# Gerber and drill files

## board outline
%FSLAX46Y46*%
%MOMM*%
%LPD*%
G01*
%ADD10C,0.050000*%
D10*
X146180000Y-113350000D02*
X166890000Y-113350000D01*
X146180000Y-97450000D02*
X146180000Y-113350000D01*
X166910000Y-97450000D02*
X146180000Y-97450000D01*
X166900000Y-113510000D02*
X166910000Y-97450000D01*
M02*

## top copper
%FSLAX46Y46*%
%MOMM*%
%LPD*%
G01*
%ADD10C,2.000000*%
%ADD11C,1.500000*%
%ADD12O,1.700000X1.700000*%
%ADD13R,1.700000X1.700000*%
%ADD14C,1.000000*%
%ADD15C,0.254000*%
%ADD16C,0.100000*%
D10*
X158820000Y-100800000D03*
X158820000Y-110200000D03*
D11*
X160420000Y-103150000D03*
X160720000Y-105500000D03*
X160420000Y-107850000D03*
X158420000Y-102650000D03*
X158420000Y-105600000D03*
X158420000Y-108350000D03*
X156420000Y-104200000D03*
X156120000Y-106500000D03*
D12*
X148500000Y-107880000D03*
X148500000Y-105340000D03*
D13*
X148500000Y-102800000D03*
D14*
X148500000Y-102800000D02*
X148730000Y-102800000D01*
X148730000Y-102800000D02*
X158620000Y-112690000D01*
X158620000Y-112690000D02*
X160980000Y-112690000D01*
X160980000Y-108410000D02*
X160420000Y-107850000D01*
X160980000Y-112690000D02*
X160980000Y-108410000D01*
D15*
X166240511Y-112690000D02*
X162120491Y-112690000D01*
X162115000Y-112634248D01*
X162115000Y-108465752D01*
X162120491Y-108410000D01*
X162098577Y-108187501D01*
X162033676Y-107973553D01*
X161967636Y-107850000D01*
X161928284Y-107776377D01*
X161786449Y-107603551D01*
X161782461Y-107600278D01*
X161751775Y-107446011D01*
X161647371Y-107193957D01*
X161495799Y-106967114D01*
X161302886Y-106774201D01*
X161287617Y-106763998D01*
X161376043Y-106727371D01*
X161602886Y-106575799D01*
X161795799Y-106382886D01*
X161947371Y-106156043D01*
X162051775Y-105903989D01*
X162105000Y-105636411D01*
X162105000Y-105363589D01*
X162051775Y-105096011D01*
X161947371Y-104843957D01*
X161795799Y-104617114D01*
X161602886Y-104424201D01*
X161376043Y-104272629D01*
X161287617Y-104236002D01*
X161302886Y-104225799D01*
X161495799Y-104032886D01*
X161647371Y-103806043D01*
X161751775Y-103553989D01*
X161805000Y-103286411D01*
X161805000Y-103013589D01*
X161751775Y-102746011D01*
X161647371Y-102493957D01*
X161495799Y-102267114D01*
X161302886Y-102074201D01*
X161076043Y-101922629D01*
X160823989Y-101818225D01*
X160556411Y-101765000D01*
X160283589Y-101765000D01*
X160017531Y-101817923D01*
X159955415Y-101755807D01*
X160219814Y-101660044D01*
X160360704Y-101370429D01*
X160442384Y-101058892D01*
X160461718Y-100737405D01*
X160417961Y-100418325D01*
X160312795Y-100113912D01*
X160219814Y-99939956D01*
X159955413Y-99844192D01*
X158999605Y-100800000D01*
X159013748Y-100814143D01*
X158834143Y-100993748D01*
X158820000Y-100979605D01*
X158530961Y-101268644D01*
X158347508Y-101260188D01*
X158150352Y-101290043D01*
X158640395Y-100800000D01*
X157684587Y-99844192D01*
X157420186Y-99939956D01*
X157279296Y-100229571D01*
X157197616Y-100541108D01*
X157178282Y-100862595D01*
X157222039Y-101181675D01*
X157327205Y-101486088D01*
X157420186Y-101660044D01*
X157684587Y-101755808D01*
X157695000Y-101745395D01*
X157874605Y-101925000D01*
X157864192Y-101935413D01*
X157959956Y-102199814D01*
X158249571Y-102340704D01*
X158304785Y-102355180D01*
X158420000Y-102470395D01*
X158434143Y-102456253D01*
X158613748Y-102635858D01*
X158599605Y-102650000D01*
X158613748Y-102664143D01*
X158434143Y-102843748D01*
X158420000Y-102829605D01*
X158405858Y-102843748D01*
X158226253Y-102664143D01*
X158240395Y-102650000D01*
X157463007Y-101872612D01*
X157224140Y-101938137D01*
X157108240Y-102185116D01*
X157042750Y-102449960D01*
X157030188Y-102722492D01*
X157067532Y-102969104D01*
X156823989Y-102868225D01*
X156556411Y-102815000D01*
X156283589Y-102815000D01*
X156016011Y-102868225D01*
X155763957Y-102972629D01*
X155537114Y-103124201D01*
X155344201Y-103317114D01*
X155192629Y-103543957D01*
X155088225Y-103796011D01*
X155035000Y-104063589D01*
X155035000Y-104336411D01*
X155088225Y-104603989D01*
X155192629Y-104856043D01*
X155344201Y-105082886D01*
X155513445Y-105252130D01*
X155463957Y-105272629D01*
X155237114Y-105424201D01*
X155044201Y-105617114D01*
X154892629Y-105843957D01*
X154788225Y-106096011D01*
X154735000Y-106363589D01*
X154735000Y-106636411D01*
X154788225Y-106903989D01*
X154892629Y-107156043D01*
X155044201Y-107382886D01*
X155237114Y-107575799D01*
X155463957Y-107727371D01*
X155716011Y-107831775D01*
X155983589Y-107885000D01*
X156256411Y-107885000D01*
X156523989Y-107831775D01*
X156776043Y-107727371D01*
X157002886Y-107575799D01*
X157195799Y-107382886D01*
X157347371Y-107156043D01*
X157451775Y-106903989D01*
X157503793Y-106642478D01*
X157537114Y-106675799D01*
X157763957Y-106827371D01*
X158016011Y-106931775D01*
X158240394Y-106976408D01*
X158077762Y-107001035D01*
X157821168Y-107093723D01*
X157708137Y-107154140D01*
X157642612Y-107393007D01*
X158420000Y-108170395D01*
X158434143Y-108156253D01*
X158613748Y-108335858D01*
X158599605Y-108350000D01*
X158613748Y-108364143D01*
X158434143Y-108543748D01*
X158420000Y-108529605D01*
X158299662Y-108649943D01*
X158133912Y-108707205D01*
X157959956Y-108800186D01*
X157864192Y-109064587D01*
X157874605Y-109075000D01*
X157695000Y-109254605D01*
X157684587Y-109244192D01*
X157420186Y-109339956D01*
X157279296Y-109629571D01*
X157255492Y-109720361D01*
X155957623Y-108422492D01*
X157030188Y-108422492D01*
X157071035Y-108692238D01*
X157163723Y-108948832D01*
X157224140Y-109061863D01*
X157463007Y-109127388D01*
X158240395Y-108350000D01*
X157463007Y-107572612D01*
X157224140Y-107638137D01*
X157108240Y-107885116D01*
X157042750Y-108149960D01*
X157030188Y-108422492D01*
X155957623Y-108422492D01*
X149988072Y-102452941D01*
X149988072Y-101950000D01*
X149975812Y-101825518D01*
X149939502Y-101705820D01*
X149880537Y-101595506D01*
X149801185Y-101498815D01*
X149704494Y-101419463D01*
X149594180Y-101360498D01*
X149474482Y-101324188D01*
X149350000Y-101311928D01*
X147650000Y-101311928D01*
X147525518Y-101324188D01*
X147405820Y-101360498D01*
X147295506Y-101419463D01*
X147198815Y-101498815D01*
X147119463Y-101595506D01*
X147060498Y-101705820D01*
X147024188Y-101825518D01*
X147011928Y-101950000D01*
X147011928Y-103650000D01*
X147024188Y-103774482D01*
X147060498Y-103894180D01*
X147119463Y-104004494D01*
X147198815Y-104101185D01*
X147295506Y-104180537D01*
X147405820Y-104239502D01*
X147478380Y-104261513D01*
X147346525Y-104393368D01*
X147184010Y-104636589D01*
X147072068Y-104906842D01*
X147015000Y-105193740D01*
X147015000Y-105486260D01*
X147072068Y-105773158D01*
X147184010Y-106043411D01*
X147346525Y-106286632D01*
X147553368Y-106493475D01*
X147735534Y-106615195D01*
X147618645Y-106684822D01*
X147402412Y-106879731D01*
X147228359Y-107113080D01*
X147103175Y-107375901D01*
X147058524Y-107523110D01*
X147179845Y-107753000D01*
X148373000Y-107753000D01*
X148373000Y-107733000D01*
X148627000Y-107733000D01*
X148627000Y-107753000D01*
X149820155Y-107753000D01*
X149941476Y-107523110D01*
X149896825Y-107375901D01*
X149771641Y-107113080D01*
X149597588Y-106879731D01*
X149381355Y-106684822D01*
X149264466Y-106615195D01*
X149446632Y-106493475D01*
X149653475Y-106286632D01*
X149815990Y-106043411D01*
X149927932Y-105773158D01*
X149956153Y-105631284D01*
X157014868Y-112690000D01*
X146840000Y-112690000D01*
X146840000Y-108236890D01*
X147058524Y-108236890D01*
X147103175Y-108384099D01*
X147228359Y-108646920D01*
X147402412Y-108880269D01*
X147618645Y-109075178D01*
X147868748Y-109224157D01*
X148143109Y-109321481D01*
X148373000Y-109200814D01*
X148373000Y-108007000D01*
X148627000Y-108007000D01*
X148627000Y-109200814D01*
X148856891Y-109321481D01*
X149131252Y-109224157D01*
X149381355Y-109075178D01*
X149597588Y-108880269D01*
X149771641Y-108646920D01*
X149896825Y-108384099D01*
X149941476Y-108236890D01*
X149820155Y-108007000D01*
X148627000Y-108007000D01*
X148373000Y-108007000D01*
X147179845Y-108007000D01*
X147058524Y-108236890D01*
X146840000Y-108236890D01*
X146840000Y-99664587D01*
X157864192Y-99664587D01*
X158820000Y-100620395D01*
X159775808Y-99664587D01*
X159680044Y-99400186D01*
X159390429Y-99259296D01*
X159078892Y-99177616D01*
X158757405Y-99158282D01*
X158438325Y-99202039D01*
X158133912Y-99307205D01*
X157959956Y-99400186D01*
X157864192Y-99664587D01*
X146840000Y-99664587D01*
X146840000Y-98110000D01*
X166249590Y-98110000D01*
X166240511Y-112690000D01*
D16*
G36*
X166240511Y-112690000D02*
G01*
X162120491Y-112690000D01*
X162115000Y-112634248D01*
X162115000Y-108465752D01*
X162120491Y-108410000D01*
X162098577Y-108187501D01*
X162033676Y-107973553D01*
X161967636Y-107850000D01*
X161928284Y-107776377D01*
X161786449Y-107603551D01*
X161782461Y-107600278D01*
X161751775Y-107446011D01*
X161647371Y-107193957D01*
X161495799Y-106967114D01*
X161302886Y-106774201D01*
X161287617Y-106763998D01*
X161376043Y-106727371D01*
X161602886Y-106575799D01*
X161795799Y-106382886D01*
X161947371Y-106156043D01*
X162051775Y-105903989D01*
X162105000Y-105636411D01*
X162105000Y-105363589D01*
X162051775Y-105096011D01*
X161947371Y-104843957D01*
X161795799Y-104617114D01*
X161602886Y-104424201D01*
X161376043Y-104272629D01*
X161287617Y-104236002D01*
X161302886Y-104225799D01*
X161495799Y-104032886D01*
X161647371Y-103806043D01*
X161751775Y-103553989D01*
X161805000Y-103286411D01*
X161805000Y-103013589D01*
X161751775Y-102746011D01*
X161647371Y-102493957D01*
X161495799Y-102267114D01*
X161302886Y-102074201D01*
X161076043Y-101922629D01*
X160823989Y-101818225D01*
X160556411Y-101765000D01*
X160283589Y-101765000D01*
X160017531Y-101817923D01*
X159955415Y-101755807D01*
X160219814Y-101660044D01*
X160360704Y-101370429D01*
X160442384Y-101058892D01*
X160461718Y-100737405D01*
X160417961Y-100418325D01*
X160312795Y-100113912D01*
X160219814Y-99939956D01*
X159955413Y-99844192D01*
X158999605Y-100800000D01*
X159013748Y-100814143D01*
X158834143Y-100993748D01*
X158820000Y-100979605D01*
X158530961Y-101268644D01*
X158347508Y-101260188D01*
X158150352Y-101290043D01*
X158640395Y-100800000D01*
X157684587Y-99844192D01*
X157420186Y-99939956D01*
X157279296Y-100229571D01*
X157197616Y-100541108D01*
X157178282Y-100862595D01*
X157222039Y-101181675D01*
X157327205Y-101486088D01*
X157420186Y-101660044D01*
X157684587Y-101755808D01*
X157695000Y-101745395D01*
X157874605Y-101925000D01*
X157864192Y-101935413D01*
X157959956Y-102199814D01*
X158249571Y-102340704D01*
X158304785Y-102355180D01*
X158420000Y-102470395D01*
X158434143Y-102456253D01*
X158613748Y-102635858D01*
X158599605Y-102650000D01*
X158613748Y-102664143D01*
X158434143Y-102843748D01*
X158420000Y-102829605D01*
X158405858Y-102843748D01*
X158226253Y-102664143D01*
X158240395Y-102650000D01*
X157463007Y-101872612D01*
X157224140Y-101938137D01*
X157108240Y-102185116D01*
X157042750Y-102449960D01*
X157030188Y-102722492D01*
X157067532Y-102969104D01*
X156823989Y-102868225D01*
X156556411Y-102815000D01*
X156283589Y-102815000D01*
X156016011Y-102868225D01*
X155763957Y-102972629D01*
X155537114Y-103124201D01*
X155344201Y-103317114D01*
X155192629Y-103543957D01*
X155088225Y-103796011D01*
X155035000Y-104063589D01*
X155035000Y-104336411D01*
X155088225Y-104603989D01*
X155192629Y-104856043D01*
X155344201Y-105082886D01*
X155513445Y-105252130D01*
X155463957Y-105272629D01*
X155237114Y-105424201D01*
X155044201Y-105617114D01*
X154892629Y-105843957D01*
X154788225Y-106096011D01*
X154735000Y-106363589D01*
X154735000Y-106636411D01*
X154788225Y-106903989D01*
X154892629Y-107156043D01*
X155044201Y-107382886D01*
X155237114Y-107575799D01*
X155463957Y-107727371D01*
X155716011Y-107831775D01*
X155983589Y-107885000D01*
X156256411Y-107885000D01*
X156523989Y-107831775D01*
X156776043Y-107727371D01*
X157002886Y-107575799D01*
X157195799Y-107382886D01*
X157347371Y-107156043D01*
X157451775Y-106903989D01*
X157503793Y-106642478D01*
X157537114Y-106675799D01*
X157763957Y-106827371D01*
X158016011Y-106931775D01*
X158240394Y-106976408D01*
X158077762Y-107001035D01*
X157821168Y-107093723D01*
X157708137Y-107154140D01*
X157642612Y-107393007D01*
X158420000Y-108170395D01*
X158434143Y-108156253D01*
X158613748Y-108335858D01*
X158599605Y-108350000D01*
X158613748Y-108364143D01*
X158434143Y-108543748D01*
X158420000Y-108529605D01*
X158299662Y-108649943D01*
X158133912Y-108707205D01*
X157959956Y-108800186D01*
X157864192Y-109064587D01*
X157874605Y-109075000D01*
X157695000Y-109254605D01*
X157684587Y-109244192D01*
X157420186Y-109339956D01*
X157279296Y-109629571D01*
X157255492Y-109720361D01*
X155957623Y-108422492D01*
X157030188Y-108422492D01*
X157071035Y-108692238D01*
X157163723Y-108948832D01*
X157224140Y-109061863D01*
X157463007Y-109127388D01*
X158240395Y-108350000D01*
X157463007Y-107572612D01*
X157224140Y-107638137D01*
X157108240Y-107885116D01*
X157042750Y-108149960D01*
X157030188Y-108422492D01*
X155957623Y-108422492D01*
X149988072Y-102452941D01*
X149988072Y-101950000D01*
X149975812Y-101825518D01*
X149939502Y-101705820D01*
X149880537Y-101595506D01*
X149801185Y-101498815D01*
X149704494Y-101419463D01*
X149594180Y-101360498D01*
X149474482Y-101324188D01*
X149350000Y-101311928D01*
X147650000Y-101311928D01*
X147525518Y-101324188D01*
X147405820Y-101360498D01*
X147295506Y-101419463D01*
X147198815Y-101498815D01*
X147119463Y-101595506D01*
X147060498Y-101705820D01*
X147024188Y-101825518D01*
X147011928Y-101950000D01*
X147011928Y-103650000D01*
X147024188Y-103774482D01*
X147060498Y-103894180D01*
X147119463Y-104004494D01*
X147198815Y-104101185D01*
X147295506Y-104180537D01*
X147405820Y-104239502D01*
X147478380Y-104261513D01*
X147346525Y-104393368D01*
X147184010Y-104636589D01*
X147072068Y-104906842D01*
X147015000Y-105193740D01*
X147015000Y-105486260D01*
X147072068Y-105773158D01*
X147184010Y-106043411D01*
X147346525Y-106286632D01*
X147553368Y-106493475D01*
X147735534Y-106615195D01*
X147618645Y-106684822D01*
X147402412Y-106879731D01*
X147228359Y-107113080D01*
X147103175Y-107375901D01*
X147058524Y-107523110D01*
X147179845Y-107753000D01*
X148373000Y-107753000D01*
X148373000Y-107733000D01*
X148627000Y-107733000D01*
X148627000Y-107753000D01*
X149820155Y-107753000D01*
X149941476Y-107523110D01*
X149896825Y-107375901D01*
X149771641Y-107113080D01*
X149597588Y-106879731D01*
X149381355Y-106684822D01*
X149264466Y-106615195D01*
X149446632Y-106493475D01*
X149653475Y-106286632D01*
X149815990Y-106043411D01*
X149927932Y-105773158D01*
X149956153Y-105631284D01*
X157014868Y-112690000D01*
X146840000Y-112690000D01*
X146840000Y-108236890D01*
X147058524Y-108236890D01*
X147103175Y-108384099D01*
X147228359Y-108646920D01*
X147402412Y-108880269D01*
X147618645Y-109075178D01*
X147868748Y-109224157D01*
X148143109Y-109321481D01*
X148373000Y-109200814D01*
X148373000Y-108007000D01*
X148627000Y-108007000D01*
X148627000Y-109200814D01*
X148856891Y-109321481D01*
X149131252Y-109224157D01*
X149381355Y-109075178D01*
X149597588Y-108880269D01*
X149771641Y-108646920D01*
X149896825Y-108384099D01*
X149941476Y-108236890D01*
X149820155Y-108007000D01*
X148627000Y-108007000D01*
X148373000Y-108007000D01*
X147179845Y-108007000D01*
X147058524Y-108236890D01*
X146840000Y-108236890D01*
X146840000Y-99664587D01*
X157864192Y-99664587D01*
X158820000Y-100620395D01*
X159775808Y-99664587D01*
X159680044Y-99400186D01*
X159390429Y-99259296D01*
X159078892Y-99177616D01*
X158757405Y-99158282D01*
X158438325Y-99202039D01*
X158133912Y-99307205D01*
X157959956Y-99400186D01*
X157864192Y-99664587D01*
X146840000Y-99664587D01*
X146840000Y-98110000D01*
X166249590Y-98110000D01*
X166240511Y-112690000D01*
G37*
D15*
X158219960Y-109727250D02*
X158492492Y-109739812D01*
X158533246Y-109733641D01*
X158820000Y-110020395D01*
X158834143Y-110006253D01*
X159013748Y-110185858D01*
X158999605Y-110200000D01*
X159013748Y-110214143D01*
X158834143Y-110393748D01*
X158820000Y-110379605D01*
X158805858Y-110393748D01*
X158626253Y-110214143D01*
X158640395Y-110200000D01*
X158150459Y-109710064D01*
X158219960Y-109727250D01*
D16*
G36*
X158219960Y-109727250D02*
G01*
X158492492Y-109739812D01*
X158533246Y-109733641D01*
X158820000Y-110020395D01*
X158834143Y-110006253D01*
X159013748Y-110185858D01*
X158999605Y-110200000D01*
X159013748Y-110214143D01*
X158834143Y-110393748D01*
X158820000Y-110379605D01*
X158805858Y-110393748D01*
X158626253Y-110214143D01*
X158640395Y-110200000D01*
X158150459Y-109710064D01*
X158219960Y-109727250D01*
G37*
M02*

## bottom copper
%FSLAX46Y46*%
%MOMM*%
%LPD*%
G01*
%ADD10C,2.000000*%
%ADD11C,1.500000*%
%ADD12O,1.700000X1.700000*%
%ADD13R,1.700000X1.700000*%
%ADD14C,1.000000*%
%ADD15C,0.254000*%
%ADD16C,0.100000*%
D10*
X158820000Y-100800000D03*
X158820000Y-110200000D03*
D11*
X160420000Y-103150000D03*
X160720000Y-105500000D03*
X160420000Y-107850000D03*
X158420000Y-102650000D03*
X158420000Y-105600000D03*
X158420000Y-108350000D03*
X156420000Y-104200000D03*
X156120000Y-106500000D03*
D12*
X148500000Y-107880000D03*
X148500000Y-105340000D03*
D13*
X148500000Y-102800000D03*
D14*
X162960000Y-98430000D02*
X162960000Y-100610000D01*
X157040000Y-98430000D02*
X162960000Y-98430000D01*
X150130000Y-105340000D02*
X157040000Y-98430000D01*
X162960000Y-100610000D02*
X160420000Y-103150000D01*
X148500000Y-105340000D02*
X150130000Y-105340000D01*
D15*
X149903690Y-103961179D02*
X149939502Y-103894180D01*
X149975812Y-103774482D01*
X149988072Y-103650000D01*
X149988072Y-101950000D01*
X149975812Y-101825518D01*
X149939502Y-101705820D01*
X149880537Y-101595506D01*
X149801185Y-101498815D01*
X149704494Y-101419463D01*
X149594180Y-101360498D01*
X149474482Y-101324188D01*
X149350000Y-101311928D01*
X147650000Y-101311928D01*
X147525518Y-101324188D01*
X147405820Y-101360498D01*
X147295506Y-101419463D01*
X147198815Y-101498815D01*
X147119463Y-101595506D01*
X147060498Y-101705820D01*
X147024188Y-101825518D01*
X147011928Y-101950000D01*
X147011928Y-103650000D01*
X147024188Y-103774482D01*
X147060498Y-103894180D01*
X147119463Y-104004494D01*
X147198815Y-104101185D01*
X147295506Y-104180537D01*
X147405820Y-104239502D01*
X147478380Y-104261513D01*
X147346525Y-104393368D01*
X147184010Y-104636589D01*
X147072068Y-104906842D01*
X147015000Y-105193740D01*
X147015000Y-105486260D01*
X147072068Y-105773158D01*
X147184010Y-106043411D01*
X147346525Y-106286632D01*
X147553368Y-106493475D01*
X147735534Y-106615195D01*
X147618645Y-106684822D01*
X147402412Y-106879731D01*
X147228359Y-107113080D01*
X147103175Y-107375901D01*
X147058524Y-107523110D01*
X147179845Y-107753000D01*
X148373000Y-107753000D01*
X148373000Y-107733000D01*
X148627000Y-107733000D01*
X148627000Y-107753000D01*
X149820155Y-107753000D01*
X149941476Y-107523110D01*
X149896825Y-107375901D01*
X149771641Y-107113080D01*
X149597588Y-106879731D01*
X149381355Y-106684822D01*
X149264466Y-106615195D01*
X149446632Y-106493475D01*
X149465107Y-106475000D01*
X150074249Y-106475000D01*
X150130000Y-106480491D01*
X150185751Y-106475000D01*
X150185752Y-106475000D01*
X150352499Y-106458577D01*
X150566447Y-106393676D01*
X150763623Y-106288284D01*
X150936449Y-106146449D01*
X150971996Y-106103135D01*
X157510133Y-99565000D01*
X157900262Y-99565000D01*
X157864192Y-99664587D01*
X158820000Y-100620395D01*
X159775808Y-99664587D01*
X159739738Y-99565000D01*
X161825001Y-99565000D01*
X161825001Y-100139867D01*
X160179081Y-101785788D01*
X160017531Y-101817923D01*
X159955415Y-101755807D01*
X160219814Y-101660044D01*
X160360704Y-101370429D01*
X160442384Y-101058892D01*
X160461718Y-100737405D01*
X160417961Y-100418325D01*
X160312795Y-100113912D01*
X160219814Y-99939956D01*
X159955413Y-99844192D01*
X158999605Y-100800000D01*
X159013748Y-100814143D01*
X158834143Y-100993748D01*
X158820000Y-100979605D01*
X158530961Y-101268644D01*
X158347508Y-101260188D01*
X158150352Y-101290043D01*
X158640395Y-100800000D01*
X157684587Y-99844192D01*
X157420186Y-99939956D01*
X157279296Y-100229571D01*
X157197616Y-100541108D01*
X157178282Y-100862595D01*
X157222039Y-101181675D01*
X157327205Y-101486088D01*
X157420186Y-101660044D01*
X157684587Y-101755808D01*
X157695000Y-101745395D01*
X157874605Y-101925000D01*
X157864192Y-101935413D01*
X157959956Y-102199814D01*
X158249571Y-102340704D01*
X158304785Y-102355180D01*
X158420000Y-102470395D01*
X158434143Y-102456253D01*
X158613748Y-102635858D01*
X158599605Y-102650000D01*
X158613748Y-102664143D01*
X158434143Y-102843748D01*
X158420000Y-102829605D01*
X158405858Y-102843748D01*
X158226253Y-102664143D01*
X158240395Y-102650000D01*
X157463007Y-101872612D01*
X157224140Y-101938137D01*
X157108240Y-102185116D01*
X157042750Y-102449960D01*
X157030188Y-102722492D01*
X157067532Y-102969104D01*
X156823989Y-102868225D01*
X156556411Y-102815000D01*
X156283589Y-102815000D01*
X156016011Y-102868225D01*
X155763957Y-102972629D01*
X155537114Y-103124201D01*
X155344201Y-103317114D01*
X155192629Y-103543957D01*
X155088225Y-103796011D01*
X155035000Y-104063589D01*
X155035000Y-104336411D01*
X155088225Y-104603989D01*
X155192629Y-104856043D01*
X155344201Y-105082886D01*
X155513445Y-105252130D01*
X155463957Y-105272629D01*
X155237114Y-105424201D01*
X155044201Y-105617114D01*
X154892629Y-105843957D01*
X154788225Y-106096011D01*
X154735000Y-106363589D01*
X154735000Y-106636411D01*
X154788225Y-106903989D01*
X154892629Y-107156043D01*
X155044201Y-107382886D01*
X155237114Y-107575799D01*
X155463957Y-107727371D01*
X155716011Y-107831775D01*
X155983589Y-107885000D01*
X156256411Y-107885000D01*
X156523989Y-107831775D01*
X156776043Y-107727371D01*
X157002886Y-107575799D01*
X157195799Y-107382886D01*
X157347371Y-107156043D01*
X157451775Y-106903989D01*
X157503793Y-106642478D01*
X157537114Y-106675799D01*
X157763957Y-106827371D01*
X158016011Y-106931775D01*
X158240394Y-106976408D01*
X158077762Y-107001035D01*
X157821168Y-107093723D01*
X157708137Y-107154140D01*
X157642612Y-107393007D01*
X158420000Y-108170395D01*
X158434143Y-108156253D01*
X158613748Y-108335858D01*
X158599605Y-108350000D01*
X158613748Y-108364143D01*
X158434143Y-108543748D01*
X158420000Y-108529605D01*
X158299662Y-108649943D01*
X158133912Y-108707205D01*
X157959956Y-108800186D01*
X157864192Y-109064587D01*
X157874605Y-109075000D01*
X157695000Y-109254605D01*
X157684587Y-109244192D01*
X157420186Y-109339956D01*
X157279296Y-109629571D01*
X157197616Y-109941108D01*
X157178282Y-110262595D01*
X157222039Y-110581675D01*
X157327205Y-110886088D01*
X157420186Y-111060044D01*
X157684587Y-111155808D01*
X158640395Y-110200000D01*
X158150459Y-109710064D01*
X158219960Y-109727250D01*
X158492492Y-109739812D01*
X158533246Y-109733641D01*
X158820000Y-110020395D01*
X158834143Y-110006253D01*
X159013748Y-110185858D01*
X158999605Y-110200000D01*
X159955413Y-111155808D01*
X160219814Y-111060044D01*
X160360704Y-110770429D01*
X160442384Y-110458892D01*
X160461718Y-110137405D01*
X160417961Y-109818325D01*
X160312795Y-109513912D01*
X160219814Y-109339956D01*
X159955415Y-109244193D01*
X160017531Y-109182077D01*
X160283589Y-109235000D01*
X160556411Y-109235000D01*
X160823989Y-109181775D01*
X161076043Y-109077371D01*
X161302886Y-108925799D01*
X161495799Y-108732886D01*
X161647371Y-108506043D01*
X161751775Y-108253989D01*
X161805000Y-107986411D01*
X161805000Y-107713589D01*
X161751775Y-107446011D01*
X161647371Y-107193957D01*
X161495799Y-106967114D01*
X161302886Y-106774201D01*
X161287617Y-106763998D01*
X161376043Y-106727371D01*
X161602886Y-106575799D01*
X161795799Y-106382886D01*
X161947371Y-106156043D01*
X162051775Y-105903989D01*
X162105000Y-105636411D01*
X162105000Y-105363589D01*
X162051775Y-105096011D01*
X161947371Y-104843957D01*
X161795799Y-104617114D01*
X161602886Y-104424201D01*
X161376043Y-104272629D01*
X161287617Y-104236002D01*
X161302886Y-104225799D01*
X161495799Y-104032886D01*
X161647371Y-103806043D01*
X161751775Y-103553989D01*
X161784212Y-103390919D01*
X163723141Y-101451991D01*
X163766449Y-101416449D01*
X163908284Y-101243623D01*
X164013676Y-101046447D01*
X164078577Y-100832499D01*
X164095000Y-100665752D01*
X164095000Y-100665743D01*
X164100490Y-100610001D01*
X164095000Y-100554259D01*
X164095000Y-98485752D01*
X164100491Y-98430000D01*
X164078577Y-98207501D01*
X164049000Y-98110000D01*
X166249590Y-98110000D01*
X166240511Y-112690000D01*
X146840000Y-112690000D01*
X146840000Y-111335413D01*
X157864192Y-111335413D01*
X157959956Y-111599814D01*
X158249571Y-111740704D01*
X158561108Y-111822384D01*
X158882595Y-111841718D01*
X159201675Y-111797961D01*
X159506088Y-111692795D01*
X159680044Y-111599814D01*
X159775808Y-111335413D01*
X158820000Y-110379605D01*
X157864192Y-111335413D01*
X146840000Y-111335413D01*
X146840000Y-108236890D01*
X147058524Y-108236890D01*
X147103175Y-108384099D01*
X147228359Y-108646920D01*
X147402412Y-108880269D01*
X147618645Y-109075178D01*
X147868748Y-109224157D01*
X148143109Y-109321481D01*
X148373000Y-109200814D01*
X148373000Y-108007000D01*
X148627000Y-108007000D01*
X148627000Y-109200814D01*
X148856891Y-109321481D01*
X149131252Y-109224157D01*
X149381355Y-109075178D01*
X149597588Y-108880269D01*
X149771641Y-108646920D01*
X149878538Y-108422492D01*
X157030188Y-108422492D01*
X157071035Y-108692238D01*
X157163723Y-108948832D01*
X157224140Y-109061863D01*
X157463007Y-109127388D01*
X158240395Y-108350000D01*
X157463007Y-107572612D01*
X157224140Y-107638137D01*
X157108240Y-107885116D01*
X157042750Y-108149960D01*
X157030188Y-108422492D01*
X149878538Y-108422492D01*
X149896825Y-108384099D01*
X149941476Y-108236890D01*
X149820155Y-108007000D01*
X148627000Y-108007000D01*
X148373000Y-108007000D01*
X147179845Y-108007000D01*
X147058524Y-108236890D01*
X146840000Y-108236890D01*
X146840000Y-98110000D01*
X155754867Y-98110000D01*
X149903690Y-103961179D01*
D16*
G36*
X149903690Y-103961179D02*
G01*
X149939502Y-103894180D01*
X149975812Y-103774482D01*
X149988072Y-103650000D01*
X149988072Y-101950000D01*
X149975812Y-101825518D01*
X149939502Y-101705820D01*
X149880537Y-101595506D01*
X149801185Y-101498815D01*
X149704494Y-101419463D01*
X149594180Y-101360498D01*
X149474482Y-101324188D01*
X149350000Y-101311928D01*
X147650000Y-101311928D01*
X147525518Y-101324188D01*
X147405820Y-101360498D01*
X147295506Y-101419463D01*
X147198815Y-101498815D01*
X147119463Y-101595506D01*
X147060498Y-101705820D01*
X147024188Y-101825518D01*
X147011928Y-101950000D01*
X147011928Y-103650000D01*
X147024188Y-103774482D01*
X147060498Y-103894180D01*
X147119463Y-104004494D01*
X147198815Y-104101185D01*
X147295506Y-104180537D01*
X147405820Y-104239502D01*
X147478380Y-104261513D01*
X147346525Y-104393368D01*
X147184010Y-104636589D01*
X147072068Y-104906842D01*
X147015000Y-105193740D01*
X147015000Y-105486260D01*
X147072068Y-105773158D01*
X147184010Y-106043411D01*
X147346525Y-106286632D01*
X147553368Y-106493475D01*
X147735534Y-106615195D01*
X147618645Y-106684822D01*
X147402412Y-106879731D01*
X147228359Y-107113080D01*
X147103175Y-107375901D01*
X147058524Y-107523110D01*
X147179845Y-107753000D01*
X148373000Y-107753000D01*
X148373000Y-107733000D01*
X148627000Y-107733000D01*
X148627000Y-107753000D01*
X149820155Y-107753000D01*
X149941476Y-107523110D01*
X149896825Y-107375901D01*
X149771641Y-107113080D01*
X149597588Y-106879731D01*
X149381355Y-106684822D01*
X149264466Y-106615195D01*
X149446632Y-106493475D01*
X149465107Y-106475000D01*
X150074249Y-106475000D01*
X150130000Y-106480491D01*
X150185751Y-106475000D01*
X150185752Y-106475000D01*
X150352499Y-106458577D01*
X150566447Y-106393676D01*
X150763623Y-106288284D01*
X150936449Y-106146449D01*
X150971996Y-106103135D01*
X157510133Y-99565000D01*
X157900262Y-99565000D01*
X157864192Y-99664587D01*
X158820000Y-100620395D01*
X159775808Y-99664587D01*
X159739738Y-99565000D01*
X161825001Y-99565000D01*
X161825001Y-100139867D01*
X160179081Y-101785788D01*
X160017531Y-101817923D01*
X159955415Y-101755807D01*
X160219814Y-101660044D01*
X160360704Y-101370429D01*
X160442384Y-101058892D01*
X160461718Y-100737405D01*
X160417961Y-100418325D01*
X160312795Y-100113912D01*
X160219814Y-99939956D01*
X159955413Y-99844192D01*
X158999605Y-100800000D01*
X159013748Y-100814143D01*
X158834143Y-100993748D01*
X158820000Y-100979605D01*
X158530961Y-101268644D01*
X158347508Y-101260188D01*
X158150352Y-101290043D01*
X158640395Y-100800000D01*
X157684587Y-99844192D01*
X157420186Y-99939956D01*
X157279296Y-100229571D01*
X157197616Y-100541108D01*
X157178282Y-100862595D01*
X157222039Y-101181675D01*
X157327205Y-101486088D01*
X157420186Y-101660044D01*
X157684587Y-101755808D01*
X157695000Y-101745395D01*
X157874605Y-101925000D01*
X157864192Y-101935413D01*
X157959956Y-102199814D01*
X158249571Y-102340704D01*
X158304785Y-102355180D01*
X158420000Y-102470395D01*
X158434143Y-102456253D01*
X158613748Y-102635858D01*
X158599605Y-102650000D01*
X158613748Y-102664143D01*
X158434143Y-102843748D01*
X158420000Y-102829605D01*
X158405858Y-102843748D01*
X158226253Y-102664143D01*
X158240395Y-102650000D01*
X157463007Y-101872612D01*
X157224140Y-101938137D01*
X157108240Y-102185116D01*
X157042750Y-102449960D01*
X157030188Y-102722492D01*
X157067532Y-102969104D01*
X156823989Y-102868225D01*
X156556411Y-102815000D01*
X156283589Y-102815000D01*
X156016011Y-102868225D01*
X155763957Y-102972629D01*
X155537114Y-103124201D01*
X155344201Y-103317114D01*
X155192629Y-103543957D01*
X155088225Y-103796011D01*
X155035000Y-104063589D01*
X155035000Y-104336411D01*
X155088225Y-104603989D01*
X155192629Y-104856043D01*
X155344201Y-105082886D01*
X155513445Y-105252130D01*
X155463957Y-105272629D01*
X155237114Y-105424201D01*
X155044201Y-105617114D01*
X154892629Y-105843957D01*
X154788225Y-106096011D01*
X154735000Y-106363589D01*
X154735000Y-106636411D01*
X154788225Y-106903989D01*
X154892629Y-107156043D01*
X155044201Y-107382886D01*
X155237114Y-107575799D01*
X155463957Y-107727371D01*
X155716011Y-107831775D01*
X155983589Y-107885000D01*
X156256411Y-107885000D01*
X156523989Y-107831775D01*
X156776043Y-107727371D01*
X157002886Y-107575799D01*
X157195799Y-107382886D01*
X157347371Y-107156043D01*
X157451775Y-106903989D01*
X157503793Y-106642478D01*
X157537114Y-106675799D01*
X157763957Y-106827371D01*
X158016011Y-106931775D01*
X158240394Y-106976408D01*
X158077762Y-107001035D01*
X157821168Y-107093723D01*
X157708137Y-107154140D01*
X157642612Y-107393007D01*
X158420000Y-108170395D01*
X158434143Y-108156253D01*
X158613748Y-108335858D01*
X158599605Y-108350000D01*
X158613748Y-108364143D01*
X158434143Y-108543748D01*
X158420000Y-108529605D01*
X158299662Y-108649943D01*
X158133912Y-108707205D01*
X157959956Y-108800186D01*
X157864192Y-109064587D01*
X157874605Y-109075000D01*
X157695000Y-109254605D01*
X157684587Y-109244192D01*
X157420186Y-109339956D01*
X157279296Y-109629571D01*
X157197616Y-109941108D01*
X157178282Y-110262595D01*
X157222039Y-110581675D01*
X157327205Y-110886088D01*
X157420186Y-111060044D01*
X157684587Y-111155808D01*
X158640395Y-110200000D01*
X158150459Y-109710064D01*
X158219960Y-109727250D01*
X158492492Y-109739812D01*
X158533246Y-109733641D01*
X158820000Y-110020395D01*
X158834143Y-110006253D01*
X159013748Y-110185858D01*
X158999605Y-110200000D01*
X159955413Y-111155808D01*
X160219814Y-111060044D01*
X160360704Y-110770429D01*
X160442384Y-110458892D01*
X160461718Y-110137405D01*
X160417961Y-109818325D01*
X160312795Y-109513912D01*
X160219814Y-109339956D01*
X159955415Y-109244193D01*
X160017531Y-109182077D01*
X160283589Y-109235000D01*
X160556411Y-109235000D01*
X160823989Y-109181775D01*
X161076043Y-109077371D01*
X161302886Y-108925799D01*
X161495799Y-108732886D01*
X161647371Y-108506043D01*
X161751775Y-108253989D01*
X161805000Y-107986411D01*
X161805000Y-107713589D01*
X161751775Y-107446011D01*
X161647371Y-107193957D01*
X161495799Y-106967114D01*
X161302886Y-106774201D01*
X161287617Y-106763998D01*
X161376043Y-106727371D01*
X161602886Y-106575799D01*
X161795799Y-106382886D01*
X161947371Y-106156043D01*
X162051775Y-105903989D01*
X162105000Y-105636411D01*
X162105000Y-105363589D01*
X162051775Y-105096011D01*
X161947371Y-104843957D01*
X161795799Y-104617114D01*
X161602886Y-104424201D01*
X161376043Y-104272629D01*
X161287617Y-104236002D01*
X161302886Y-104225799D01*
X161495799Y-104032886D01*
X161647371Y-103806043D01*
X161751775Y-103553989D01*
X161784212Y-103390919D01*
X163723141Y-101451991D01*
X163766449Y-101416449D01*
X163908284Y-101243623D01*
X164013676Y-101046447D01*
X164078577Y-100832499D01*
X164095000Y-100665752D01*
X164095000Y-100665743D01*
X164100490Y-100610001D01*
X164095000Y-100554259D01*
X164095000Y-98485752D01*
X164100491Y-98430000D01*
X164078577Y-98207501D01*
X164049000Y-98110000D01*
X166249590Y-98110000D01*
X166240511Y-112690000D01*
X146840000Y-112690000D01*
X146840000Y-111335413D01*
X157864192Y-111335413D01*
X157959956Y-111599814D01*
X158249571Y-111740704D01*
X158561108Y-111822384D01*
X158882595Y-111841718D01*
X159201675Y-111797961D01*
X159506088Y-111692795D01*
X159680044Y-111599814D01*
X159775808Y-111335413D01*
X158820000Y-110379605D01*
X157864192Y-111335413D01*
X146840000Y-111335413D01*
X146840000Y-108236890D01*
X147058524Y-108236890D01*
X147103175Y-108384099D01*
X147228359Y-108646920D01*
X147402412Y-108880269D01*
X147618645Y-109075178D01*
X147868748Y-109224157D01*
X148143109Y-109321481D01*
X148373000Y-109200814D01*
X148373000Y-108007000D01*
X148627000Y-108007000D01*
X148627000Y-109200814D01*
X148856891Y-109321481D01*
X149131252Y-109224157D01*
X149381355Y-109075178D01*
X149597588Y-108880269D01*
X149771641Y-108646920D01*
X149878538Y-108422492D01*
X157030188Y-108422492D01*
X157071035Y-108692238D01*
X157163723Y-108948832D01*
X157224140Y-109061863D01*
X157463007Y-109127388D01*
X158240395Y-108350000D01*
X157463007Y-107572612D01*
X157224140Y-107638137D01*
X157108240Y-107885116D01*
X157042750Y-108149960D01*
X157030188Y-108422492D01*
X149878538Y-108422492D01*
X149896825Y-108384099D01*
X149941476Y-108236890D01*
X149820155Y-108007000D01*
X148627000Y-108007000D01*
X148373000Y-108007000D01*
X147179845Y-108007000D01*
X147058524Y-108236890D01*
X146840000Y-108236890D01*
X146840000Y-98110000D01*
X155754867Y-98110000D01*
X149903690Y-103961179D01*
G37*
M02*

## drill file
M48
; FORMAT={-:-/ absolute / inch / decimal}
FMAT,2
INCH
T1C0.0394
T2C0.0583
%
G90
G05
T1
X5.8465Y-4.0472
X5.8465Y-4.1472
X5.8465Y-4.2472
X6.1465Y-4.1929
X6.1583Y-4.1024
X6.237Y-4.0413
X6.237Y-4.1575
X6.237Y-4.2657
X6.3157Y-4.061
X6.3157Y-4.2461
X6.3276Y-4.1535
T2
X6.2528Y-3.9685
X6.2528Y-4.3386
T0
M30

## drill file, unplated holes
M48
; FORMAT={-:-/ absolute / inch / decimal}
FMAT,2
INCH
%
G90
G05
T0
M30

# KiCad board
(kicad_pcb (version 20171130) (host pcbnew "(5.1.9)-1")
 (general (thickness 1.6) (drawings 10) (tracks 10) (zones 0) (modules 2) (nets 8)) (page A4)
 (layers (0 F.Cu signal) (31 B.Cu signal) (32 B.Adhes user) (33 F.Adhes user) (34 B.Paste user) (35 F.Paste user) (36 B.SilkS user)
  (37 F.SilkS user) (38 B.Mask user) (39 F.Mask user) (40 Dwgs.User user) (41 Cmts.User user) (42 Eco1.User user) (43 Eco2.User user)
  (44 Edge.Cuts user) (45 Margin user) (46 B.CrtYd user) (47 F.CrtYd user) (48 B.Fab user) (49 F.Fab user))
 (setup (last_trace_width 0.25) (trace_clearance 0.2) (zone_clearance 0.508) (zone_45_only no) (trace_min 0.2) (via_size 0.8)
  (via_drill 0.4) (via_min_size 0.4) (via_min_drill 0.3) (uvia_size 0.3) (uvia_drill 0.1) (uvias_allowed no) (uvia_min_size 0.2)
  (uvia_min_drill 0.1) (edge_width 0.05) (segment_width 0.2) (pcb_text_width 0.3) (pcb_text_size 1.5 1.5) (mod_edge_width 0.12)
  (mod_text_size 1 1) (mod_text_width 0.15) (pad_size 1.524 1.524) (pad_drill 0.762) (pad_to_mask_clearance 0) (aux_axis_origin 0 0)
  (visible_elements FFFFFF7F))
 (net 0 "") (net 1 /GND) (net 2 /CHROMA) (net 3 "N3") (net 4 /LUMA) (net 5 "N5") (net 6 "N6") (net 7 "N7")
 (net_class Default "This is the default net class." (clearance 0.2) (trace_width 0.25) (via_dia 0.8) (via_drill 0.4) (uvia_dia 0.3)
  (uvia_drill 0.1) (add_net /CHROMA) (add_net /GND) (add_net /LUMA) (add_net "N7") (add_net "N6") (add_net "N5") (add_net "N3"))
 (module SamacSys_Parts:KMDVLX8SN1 (layer F.Cu) (at 156.12 106.5 90)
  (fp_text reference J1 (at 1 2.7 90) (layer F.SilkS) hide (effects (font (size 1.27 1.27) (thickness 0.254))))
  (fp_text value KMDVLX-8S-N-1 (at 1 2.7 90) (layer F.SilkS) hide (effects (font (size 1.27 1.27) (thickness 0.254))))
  (pad MH2 thru_hole circle (at 5.7 2.7 180) (size 2 2) (drill 1.48) (layers *.Cu *.Mask F.SilkS) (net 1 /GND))
  (pad MH1 thru_hole circle (at -3.7 2.7 180) (size 2 2) (drill 1.48) (layers *.Cu *.Mask F.SilkS) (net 1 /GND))
  (pad 8 thru_hole circle (at 3.35 4.3 180) (size 1.5 1.5) (drill 1) (layers *.Cu *.Mask F.SilkS) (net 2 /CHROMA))
  (pad 7 thru_hole circle (at 1 4.6 180) (size 1.5 1.5) (drill 1) (layers *.Cu *.Mask F.SilkS) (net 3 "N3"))
  (pad 6 thru_hole circle (at -1.35 4.3 180) (size 1.5 1.5) (drill 1) (layers *.Cu *.Mask F.SilkS) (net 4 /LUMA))
  (pad 5 thru_hole circle (at 3.85 2.3 180) (size 1.5 1.5) (drill 1) (layers *.Cu *.Mask F.SilkS) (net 1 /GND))
  (pad 4 thru_hole circle (at 0.9 2.3 180) (size 1.5 1.5) (drill 1) (layers *.Cu *.Mask F.SilkS) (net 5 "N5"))
  (pad 3 thru_hole circle (at -1.85 2.3 180) (size 1.5 1.5) (drill 1) (layers *.Cu *.Mask F.SilkS) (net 1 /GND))
  (pad 2 thru_hole circle (at 2.3 0.3 180) (size 1.5 1.5) (drill 1) (layers *.Cu *.Mask F.SilkS) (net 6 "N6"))
  (pad 1 thru_hole circle (at 0 0 180) (size 1.5 1.5) (drill 1) (layers *.Cu *.Mask F.SilkS) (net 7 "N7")))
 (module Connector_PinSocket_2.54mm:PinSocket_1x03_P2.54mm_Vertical (layer F.Cu) (at 148.5 102.8)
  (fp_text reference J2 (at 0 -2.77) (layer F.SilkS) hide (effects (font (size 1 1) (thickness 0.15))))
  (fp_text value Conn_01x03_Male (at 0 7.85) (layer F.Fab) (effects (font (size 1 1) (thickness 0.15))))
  (pad 3 thru_hole oval (at 0 5.08) (size 1.7 1.7) (drill 1) (layers *.Cu *.Mask) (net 1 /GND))
  (pad 2 thru_hole oval (at 0 2.54) (size 1.7 1.7) (drill 1) (layers *.Cu *.Mask) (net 2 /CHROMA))
  (pad 1 thru_hole rect (at 0 0) (size 1.7 1.7) (drill 1) (layers *.Cu *.Mask) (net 4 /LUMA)))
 (gr_line (start 146.18 113.35) (end 166.89 113.35) (layer Edge.Cuts) (width 0.05))
 (gr_line (start 146.18 97.45) (end 146.18 113.35) (layer Edge.Cuts) (width 0.05))
 (gr_line (start 166.91 97.45) (end 146.18 97.45) (layer Edge.Cuts) (width 0.05))
 (gr_line (start 166.9 113.51) (end 166.91 97.45) (layer Edge.Cuts) (width 0.05))
 (segment (start 162.96 98.43) (end 162.96 100.61) (width 1) (layer B.Cu) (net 2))
 (segment (start 157.04 98.43) (end 162.96 98.43) (width 1) (layer B.Cu) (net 2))
 (segment (start 150.13 105.34) (end 157.04 98.43) (width 1) (layer B.Cu) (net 2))
 (segment (start 162.96 100.61) (end 160.42 103.15) (width 1) (layer B.Cu) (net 2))
 (segment (start 148.5 105.34) (end 150.13 105.34) (width 1) (layer B.Cu) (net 2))
 (segment (start 148.5 102.8) (end 148.73 102.8) (width 1) (layer F.Cu) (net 4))
 (segment (start 148.73 102.8) (end 158.62 112.69) (width 1) (layer F.Cu) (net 4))
 (segment (start 158.62 112.69) (end 160.98 112.69) (width 1) (layer F.Cu) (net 4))
 (segment (start 160.98 108.41) (end 160.42 107.85) (width 1) (layer F.Cu) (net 4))
 (segment (start 160.98 112.69) (end 160.98 108.41) (width 1) (layer F.Cu) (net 4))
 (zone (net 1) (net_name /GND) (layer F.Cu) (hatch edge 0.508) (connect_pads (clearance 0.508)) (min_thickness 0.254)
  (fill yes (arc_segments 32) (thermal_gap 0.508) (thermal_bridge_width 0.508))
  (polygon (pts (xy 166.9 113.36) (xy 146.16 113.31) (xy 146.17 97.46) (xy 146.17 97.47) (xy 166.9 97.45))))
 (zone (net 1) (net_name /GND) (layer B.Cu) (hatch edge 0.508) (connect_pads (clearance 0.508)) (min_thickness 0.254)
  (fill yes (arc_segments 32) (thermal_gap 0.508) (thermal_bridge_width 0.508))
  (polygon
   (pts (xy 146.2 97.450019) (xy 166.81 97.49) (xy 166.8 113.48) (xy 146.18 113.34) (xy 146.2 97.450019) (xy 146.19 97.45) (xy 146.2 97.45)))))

